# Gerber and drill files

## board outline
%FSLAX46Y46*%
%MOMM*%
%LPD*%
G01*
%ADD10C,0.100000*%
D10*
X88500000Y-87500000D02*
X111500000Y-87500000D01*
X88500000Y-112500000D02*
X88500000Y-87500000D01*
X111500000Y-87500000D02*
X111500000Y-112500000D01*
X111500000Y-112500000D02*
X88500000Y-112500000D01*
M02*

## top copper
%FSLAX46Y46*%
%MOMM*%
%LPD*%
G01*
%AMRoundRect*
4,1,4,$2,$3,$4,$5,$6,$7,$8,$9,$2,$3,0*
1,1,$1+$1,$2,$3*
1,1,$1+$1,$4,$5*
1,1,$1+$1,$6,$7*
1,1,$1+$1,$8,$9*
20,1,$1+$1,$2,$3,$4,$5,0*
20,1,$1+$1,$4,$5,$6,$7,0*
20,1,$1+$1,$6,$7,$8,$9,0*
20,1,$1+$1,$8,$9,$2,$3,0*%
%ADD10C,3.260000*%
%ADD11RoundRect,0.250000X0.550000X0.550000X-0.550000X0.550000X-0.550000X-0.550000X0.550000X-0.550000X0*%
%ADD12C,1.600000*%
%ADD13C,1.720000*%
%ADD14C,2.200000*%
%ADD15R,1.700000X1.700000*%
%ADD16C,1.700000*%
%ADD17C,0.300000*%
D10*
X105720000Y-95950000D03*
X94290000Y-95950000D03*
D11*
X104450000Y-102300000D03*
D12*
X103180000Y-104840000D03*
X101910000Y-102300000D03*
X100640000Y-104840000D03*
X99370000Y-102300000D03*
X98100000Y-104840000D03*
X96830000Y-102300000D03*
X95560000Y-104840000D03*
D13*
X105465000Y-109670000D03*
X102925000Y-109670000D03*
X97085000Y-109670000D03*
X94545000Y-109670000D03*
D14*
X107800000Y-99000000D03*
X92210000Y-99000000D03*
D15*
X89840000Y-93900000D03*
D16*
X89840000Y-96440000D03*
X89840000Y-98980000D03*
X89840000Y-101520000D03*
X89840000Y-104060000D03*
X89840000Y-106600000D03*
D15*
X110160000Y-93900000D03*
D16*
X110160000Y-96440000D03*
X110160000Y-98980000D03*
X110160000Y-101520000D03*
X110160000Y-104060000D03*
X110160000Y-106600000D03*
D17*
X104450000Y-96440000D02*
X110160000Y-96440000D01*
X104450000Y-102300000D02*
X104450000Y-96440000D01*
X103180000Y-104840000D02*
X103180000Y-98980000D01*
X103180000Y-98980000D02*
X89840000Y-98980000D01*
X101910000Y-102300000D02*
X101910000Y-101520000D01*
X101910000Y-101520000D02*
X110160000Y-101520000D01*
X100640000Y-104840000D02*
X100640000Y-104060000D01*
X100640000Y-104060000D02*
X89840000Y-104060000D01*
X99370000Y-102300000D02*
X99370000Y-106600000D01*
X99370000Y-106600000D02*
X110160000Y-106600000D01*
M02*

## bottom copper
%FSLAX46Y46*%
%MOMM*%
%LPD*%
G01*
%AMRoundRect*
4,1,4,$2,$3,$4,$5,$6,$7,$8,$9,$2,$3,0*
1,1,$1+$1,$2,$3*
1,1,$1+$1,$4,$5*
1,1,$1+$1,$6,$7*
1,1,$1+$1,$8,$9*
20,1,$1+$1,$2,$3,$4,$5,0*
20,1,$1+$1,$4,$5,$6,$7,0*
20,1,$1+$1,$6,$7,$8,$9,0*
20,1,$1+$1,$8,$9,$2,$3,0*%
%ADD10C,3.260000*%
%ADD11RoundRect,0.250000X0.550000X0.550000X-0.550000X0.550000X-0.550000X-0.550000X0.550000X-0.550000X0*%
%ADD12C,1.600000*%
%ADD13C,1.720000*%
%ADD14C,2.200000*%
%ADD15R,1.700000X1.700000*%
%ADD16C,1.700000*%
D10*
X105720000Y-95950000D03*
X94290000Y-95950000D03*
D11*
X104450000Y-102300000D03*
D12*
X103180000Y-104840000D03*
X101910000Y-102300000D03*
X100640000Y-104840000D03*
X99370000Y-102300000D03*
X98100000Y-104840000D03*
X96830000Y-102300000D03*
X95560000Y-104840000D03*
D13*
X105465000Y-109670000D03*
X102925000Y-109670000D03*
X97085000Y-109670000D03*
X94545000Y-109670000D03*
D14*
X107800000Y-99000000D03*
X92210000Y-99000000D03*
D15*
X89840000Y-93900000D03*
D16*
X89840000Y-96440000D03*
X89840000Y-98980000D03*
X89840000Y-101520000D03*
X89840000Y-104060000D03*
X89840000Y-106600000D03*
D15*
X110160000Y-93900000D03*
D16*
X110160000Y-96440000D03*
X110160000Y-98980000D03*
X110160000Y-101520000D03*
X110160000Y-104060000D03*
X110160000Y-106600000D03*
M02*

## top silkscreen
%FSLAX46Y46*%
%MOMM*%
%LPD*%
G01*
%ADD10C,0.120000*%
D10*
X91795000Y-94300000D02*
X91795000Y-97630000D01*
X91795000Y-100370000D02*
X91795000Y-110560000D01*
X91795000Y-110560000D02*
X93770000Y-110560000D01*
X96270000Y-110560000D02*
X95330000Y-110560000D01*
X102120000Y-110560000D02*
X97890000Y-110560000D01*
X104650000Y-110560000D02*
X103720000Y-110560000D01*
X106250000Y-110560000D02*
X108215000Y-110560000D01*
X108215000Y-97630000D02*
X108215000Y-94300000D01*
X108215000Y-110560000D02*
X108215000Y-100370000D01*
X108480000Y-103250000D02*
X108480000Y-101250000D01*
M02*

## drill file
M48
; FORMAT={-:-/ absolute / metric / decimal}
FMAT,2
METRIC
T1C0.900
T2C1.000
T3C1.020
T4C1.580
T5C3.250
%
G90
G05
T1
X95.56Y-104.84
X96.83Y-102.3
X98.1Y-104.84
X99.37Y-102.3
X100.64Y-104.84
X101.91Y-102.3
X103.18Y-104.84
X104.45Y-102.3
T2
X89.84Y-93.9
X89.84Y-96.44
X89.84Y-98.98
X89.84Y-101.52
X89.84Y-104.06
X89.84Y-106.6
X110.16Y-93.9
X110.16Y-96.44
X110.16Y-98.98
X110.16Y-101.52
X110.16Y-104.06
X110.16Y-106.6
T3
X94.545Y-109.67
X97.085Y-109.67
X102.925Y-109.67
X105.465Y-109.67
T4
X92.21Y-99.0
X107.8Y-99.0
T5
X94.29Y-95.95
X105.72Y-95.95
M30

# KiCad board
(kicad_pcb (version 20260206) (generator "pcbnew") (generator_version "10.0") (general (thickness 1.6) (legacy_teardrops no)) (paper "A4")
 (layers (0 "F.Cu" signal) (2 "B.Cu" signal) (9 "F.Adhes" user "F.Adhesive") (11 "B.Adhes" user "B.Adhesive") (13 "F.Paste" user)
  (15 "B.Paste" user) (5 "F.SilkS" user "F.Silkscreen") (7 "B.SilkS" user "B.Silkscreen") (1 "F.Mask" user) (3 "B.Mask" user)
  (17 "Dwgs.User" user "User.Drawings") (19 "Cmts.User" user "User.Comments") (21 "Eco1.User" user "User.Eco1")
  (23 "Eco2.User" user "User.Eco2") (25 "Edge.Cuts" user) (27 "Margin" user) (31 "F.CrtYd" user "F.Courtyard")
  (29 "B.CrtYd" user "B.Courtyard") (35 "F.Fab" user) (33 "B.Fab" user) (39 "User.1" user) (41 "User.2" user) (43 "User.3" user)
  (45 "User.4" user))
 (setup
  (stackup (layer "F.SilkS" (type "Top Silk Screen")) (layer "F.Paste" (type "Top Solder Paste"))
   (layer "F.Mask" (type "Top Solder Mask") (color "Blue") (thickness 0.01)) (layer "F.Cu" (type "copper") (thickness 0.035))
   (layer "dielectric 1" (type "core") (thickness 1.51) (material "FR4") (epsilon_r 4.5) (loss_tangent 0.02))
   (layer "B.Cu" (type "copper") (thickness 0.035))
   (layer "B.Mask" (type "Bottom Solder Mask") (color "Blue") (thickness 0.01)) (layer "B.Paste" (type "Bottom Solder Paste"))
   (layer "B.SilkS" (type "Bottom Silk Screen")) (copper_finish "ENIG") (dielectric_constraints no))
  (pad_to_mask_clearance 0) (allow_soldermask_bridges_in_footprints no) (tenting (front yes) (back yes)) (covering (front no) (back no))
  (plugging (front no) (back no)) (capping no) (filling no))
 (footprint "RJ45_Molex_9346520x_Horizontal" (layer "F.Cu") (at 104.45 102.3 180)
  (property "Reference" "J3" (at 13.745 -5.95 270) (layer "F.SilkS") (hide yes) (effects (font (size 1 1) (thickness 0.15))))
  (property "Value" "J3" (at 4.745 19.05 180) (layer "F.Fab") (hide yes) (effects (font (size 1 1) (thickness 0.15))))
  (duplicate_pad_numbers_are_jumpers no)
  (fp_line (start 12.655 8) (end 12.655 4.67) (stroke (width 0.12) (type solid)) (layer "F.SilkS"))
  (fp_line (start 12.655 1.93) (end 12.655 -8.26) (stroke (width 0.12) (type solid)) (layer "F.SilkS"))
  (fp_line (start 12.655 -8.26) (end 10.68 -8.26) (stroke (width 0.12) (type solid)) (layer "F.SilkS"))
  (fp_line (start 8.18 -8.26) (end 9.12 -8.26) (stroke (width 0.12) (type solid)) (layer "F.SilkS"))
  (fp_line (start 2.33 -8.26) (end 6.56 -8.26) (stroke (width 0.12) (type solid)) (layer "F.SilkS"))
  (fp_line (start -0.2 -8.26) (end 0.73 -8.26) (stroke (width 0.12) (type solid)) (layer "F.SilkS"))
  (fp_line (start -1.8 -8.26) (end -3.765 -8.26) (stroke (width 0.12) (type solid)) (layer "F.SilkS"))
  (fp_line (start -3.765 4.67) (end -3.765 8) (stroke (width 0.12) (type solid)) (layer "F.SilkS"))
  (fp_line (start -3.765 -8.26) (end -3.765 1.93) (stroke (width 0.12) (type solid)) (layer "F.SilkS"))
  (fp_line (start -4.03 -0.95) (end -4.03 1.05) (stroke (width 0.12) (type solid)) (layer "F.SilkS"))
  (pad "" np_thru_hole circle (at -1.27 6.35 180) (size 3.26 3.26) (drill 3.25) (layers "*.Cu" "*.Mask"))
  (pad "" np_thru_hole circle (at 10.16 6.35 180) (size 3.26 3.26) (drill 3.25) (layers "*.Cu" "*.Mask"))
  (pad "2" thru_hole roundrect (at 0 0 180) (size 1.6 1.6) (drill 0.9) (layers "*.Cu" "*.Mask") (remove_unused_layers no)
   (roundrect_rratio 0.15625) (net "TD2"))
  (pad "3" thru_hole circle (at 1.27 -2.54 180) (size 1.6 1.6) (drill 0.9) (layers "*.Cu" "*.Mask") (remove_unused_layers no) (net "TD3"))
  (pad "4" thru_hole circle (at 2.54 0 180) (size 1.6 1.6) (drill 0.9) (layers "*.Cu" "*.Mask") (remove_unused_layers no) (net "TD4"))
  (pad "5" thru_hole circle (at 3.81 -2.54 180) (size 1.6 1.6) (drill 0.9) (layers "*.Cu" "*.Mask") (remove_unused_layers no) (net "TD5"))
  (pad "6" thru_hole circle (at 5.08 0 180) (size 1.6 1.6) (drill 0.9) (layers "*.Cu" "*.Mask") (remove_unused_layers no) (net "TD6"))
  (pad "7" thru_hole circle (at 6.35 -2.54 180) (size 1.6 1.6) (drill 0.9) (layers "*.Cu" "*.Mask") (remove_unused_layers no) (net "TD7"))
  (pad "8" thru_hole circle (at 7.62 0 180) (size 1.6 1.6) (drill 0.9) (layers "*.Cu" "*.Mask") (remove_unused_layers no) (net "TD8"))
  (pad "9" thru_hole circle (at 8.89 -2.54 180) (size 1.6 1.6) (drill 0.9) (layers "*.Cu" "*.Mask") (remove_unused_layers no))
  (pad "11" thru_hole circle (at -1.015 -7.37 180) (size 1.72 1.72) (drill 1.02) (layers "*.Cu" "*.Mask") (remove_unused_layers no))
  (pad "12" thru_hole circle (at 1.525 -7.37 180) (size 1.72 1.72) (drill 1.02) (layers "*.Cu" "*.Mask") (remove_unused_layers no))
  (pad "13" thru_hole circle (at 7.365 -7.37 180) (size 1.72 1.72) (drill 1.02) (layers "*.Cu" "*.Mask") (remove_unused_layers no))
  (pad "14" thru_hole circle (at 9.905 -7.37 180) (size 1.72 1.72) (drill 1.02) (layers "*.Cu" "*.Mask") (remove_unused_layers no))
  (pad "SH" thru_hole circle (at -3.35 3.3 180) (size 2.2 2.2) (drill 1.58) (layers "*.Cu" "*.Mask") (remove_unused_layers no))
  (pad "SH" thru_hole circle (at 12.24 3.3 180) (size 2.2 2.2) (drill 1.58) (layers "*.Cu" "*.Mask") (remove_unused_layers no))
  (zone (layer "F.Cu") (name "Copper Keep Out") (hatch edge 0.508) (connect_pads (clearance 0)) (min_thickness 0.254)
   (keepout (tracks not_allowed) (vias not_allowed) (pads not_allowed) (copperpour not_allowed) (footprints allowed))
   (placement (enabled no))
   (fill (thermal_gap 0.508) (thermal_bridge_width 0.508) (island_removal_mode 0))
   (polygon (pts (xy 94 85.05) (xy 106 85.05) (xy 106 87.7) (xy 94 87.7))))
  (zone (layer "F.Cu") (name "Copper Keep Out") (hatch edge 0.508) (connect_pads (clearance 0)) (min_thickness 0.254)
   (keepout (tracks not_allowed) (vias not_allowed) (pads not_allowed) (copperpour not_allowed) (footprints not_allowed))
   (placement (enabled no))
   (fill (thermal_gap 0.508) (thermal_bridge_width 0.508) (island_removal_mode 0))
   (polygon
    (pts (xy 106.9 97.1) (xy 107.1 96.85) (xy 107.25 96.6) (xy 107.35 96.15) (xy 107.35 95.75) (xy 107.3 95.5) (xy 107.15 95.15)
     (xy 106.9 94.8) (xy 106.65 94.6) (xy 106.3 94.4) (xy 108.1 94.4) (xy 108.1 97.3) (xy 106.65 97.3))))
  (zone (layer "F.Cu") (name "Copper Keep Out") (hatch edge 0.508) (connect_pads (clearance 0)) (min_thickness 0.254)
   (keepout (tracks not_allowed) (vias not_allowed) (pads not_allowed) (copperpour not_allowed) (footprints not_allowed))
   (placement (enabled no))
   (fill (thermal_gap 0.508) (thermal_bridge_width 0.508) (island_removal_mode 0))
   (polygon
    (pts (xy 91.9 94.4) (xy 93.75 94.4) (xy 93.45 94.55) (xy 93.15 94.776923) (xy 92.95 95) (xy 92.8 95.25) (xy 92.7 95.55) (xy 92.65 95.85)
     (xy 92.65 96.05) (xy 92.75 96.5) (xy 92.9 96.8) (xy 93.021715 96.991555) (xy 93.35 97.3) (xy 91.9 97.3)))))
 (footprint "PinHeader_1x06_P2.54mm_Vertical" (layer "B.Cu") (at 89.84 93.9 180)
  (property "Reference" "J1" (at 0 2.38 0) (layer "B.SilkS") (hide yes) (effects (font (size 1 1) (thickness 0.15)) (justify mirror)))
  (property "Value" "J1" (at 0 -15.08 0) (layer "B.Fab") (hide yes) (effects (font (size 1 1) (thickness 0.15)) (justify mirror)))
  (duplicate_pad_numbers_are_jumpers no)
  (pad "1" thru_hole rect (at 0 0 180) (size 1.7 1.7) (drill 1) (layers "*.Cu" "*.Mask") (remove_unused_layers no) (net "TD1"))
  (pad "2" thru_hole circle (at 0 -2.54 180) (size 1.7 1.7) (drill 1) (layers "*.Cu" "*.Mask") (remove_unused_layers no) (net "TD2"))
  (pad "3" thru_hole circle (at 0 -5.08 180) (size 1.7 1.7) (drill 1) (layers "*.Cu" "*.Mask") (remove_unused_layers no) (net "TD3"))
  (pad "4" thru_hole circle (at 0 -7.62 180) (size 1.7 1.7) (drill 1) (layers "*.Cu" "*.Mask") (remove_unused_layers no) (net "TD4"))
  (pad "5" thru_hole circle (at 0 -10.16 180) (size 1.7 1.7) (drill 1) (layers "*.Cu" "*.Mask") (remove_unused_layers no) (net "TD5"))
  (pad "6" thru_hole circle (at 0 -12.7 180) (size 1.7 1.7) (drill 1) (layers "*.Cu" "*.Mask") (remove_unused_layers no) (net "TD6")))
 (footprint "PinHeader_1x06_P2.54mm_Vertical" (layer "B.Cu") (at 110.16 93.9 180)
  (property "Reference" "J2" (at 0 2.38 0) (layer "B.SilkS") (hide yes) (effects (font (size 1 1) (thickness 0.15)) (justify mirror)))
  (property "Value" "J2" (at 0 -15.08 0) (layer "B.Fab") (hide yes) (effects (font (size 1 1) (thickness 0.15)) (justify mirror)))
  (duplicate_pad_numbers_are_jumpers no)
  (pad "1" thru_hole rect (at 0 0 180) (size 1.7 1.7) (drill 1) (layers "*.Cu" "*.Mask") (remove_unused_layers no) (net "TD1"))
  (pad "2" thru_hole circle (at 0 -2.54 180) (size 1.7 1.7) (drill 1) (layers "*.Cu" "*.Mask") (remove_unused_layers no) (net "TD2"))
  (pad "3" thru_hole circle (at 0 -5.08 180) (size 1.7 1.7) (drill 1) (layers "*.Cu" "*.Mask") (remove_unused_layers no) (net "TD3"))
  (pad "4" thru_hole circle (at 0 -7.62 180) (size 1.7 1.7) (drill 1) (layers "*.Cu" "*.Mask") (remove_unused_layers no) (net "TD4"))
  (pad "5" thru_hole circle (at 0 -10.16 180) (size 1.7 1.7) (drill 1) (layers "*.Cu" "*.Mask") (remove_unused_layers no) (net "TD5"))
  (pad "6" thru_hole circle (at 0 -12.7 180) (size 1.7 1.7) (drill 1) (layers "*.Cu" "*.Mask") (remove_unused_layers no) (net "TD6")))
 (gr_line (start 88.5 87.5) (end 111.5 87.5) (stroke (width 0.1) (type default)) (layer "Edge.Cuts"))
 (gr_line (start 88.5 112.5) (end 88.5 87.5) (stroke (width 0.1) (type default)) (layer "Edge.Cuts"))
 (gr_line (start 111.5 87.5) (end 111.5 112.5) (stroke (width 0.1) (type default)) (layer "Edge.Cuts"))
 (gr_line (start 111.5 112.5) (end 88.5 112.5) (stroke (width 0.1) (type default)) (layer "Edge.Cuts"))
 (segment (start 104.45 96.44) (end 110.16 96.44) (width 0.3) (layer "F.Cu") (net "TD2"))
 (segment (start 104.45 102.3) (end 104.45 96.44) (width 0.3) (layer "F.Cu") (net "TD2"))
 (segment (start 103.18 104.84) (end 103.18 98.98) (width 0.3) (layer "F.Cu") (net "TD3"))
 (segment (start 103.18 98.98) (end 89.84 98.98) (width 0.3) (layer "F.Cu") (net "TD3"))
 (segment (start 101.91 102.3) (end 101.91 101.52) (width 0.3) (layer "F.Cu") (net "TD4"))
 (segment (start 101.91 101.52) (end 110.16 101.52) (width 0.3) (layer "F.Cu") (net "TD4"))
 (segment (start 100.64 104.84) (end 100.64 104.06) (width 0.3) (layer "F.Cu") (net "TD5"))
 (segment (start 100.64 104.06) (end 89.84 104.06) (width 0.3) (layer "F.Cu") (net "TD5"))
 (segment (start 99.37 102.3) (end 99.37 106.6) (width 0.3) (layer "F.Cu") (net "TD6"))
 (segment (start 99.37 106.6) (end 110.16 106.6) (width 0.3) (layer "F.Cu") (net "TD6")))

